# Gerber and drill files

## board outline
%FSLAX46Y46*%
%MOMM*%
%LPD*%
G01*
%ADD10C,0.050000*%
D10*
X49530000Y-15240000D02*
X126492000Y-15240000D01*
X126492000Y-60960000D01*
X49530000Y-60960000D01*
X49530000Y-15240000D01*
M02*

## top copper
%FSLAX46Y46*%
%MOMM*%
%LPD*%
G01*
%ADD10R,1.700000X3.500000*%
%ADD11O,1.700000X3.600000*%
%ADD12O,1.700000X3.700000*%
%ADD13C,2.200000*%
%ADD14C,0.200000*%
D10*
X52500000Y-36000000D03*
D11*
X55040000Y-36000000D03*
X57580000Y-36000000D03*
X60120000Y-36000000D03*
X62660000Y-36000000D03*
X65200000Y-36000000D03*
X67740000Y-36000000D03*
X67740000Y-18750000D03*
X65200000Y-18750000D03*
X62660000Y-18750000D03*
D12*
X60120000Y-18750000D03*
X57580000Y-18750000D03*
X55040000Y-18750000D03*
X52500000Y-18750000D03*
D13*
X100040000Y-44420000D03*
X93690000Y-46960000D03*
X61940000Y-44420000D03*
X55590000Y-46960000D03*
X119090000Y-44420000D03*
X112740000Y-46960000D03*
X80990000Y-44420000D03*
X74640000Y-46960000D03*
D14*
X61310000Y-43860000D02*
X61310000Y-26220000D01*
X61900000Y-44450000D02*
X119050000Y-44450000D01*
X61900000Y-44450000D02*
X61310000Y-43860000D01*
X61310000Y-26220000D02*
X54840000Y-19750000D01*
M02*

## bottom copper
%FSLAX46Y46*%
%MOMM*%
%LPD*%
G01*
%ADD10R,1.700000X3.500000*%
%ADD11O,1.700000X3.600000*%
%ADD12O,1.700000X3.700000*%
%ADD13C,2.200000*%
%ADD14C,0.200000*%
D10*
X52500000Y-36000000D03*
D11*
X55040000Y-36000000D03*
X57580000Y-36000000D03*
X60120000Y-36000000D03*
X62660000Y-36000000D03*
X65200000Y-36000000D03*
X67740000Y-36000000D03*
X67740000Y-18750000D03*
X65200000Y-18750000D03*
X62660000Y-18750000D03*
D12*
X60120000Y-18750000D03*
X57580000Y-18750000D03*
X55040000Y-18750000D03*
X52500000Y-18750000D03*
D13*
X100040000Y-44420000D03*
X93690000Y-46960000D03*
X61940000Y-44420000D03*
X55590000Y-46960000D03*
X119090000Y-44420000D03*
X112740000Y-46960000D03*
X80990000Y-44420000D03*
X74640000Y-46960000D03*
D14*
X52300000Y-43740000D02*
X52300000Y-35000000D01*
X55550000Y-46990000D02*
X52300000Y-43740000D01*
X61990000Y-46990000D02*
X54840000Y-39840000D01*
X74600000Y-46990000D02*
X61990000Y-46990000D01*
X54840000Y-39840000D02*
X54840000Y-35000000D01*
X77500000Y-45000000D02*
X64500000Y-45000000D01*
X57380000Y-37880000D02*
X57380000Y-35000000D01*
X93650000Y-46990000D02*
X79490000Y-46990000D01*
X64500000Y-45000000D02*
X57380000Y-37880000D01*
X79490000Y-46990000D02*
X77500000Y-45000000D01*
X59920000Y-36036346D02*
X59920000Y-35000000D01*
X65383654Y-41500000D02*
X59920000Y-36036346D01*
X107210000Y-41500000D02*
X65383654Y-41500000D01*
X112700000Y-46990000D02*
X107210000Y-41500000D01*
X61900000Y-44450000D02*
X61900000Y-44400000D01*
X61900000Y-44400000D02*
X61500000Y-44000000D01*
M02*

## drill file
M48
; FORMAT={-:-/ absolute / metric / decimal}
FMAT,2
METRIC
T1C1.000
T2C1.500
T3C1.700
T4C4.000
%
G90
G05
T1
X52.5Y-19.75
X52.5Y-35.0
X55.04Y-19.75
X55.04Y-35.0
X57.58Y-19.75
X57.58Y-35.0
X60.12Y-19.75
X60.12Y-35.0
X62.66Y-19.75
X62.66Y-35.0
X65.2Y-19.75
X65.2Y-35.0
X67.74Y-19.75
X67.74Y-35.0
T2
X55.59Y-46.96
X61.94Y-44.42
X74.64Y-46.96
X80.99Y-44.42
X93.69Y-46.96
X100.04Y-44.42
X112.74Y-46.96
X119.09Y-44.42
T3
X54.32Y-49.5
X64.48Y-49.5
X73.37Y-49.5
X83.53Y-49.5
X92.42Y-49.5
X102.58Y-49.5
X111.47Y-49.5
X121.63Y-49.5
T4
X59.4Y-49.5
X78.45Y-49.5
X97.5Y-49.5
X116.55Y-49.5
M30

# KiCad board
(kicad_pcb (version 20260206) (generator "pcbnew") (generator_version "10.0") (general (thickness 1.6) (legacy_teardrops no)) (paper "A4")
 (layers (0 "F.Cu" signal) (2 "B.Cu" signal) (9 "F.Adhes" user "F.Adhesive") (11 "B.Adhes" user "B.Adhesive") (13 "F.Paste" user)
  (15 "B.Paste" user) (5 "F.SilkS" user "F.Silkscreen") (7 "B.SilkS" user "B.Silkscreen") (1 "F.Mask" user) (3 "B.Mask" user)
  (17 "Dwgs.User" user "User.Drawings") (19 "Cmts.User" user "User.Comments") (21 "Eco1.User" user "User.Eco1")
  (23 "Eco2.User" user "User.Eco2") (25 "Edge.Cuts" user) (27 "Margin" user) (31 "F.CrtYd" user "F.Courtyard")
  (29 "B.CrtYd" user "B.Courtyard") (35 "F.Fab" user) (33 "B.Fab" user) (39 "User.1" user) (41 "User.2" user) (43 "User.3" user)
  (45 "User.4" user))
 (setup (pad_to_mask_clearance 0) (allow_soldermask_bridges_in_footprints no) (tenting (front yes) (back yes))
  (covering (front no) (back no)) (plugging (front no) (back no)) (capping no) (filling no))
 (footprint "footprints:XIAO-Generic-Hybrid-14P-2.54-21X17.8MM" (layer "F.Cu") (at 60.12 27.375 90)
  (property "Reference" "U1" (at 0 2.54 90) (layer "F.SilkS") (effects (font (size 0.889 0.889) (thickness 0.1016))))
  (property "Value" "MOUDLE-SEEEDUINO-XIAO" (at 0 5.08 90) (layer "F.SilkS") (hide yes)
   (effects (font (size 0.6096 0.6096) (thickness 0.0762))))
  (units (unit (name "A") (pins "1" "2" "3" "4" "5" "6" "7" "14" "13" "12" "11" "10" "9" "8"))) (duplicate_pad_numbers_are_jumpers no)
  (pad "1" thru_hole rect (at -7.625 -7.62 90) (size 3.5 1.7) (drill 1 (offset -1 0)) (layers "*.Cu" "*.Mask") (remove_unused_layers no)
   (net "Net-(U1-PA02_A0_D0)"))
  (pad "2" thru_hole oval (at -7.625 -5.08 90) (size 3.6 1.7) (drill 1 (offset -1 0)) (layers "*.Cu" "*.Mask") (remove_unused_layers no)
   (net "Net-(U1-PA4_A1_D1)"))
  (pad "3" thru_hole oval (at -7.625 -2.54 90) (size 3.6 1.7) (drill 1 (offset -1 0)) (layers "*.Cu" "*.Mask") (remove_unused_layers no)
   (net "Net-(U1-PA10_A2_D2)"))
  (pad "4" thru_hole oval (at -7.625 0 90) (size 3.6 1.7) (drill 1 (offset -1 0)) (layers "*.Cu" "*.Mask") (remove_unused_layers no)
   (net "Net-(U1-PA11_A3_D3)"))
  (pad "5" thru_hole oval (at -7.625 2.54 90) (size 3.6 1.7) (drill 1 (offset -1 0)) (layers "*.Cu" "*.Mask") (remove_unused_layers no)
   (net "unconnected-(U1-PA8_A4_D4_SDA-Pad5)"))
  (pad "6" thru_hole oval (at -7.625 5.08 270) (size 3.6 1.7) (drill 1 (offset 1 0)) (layers "*.Cu" "*.Mask") (remove_unused_layers no)
   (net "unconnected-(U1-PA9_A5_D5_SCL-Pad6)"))
  (pad "7" thru_hole oval (at -7.625 7.62 90) (size 3.6 1.7) (drill 1 (offset -1 0)) (layers "*.Cu" "*.Mask") (remove_unused_layers no)
   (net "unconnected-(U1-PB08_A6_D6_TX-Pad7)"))
  (pad "8" thru_hole oval (at 7.625 7.62 90) (size 3.6 1.7) (drill 1 (offset 1 0)) (layers "*.Cu" "*.Mask") (remove_unused_layers no)
   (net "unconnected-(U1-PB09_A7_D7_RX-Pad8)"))
  (pad "9" thru_hole oval (at 7.625 5.08 90) (size 3.6 1.7) (drill 1 (offset 1 0)) (layers "*.Cu" "*.Mask") (remove_unused_layers no)
   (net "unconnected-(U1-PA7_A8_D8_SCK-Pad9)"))
  (pad "10" thru_hole oval (at 7.625 2.54 90) (size 3.6 1.7) (drill 1 (offset 1 0)) (layers "*.Cu" "*.Mask") (remove_unused_layers no)
   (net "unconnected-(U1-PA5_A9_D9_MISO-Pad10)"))
  (pad "11" thru_hole oval (at 7.625 0 90) (size 3.7 1.7) (drill 1 (offset 1 0)) (layers "*.Cu" "*.Mask") (remove_unused_layers no)
   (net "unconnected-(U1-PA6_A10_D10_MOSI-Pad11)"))
  (pad "12" thru_hole oval (at 7.625 -2.54 90) (size 3.7 1.7) (drill 1 (offset 1 0)) (layers "*.Cu" "*.Mask") (remove_unused_layers no)
   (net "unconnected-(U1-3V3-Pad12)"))
  (pad "13" thru_hole oval (at 7.625 -5.08 90) (size 3.7 1.7) (drill 1 (offset 1 0)) (layers "*.Cu" "*.Mask") (remove_unused_layers no)
   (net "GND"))
  (pad "14" thru_hole oval (at 7.625 -7.62 90) (size 3.7 1.7) (drill 1 (offset 1 0)) (layers "*.Cu" "*.Mask") (remove_unused_layers no)
   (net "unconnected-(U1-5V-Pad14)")))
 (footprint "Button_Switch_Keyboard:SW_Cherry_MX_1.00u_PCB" (layer "F.Cu") (at 100.04 44.42)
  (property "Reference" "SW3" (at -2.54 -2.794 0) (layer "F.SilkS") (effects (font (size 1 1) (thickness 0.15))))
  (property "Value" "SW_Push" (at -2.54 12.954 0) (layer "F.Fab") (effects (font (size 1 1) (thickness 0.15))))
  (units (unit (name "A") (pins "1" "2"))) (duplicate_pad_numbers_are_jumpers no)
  (pad "" np_thru_hole circle (at -7.62 5.08) (size 1.7 1.7) (drill 1.7) (layers "*.Cu" "*.Mask"))
  (pad "" np_thru_hole circle (at -2.54 5.08) (size 4 4) (drill 4) (layers "*.Cu" "*.Mask"))
  (pad "" np_thru_hole circle (at 2.54 5.08) (size 1.7 1.7) (drill 1.7) (layers "*.Cu" "*.Mask"))
  (pad "1" thru_hole circle (at 0 0) (size 2.2 2.2) (drill 1.5) (layers "*.Cu" "*.Mask") (remove_unused_layers no) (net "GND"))
  (pad "2" thru_hole circle (at -6.35 2.54) (size 2.2 2.2) (drill 1.5) (layers "*.Cu" "*.Mask") (remove_unused_layers no)
   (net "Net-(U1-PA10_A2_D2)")))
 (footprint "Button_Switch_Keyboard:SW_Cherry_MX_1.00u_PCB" (layer "F.Cu") (at 61.94 44.42)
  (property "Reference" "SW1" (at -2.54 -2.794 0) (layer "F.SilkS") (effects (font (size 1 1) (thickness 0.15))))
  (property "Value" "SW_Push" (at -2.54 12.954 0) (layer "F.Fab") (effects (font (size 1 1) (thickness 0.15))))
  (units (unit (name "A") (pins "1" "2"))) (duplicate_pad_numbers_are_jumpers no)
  (pad "" np_thru_hole circle (at -7.62 5.08) (size 1.7 1.7) (drill 1.7) (layers "*.Cu" "*.Mask"))
  (pad "" np_thru_hole circle (at -2.54 5.08) (size 4 4) (drill 4) (layers "*.Cu" "*.Mask"))
  (pad "" np_thru_hole circle (at 2.54 5.08) (size 1.7 1.7) (drill 1.7) (layers "*.Cu" "*.Mask"))
  (pad "1" thru_hole circle (at 0 0) (size 2.2 2.2) (drill 1.5) (layers "*.Cu" "*.Mask") (remove_unused_layers no) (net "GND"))
  (pad "2" thru_hole circle (at -6.35 2.54) (size 2.2 2.2) (drill 1.5) (layers "*.Cu" "*.Mask") (remove_unused_layers no)
   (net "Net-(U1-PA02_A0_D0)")))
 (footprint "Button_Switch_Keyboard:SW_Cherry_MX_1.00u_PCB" (layer "F.Cu") (at 119.09 44.42)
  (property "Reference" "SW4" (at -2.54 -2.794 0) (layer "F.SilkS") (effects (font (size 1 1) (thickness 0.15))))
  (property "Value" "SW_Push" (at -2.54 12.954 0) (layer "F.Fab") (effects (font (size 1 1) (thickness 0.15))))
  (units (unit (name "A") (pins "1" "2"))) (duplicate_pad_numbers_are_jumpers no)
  (pad "" np_thru_hole circle (at -7.62 5.08) (size 1.7 1.7) (drill 1.7) (layers "*.Cu" "*.Mask"))
  (pad "" np_thru_hole circle (at -2.54 5.08) (size 4 4) (drill 4) (layers "*.Cu" "*.Mask"))
  (pad "" np_thru_hole circle (at 2.54 5.08) (size 1.7 1.7) (drill 1.7) (layers "*.Cu" "*.Mask"))
  (pad "1" thru_hole circle (at 0 0) (size 2.2 2.2) (drill 1.5) (layers "*.Cu" "*.Mask") (remove_unused_layers no) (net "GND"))
  (pad "2" thru_hole circle (at -6.35 2.54) (size 2.2 2.2) (drill 1.5) (layers "*.Cu" "*.Mask") (remove_unused_layers no)
   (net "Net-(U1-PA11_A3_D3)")))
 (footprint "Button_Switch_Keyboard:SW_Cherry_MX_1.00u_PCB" (layer "F.Cu") (at 80.99 44.42)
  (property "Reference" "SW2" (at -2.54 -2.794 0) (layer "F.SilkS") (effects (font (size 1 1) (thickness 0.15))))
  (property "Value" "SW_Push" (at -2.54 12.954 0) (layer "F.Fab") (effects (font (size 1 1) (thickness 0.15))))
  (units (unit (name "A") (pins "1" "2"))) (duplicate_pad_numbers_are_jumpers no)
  (pad "" np_thru_hole circle (at -7.62 5.08) (size 1.7 1.7) (drill 1.7) (layers "*.Cu" "*.Mask"))
  (pad "" np_thru_hole circle (at -2.54 5.08) (size 4 4) (drill 4) (layers "*.Cu" "*.Mask"))
  (pad "" np_thru_hole circle (at 2.54 5.08) (size 1.7 1.7) (drill 1.7) (layers "*.Cu" "*.Mask"))
  (pad "1" thru_hole circle (at 0 0) (size 2.2 2.2) (drill 1.5) (layers "*.Cu" "*.Mask") (remove_unused_layers no) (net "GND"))
  (pad "2" thru_hole circle (at -6.35 2.54) (size 2.2 2.2) (drill 1.5) (layers "*.Cu" "*.Mask") (remove_unused_layers no)
   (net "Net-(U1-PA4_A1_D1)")))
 (gr_rect (start 49.53 15.24) (end 126.492 60.96) (stroke (width 0.05) (type solid)) (fill no) (layer "Edge.Cuts"))
 (segment (start 52.3 43.74) (end 52.3 35) (width 0.2) (layer "B.Cu") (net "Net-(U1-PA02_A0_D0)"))
 (segment (start 55.55 46.99) (end 52.3 43.74) (width 0.2) (layer "B.Cu") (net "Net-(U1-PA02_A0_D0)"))
 (segment (start 61.99 46.99) (end 54.84 39.84) (width 0.2) (layer "B.Cu") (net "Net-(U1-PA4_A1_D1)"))
 (segment (start 74.6 46.99) (end 61.99 46.99) (width 0.2) (layer "B.Cu") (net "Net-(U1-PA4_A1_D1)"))
 (segment (start 54.84 39.84) (end 54.84 35) (width 0.2) (layer "B.Cu") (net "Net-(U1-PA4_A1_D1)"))
 (segment (start 77.5 45) (end 64.5 45) (width 0.2) (layer "B.Cu") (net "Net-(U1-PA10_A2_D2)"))
 (segment (start 57.38 37.88) (end 57.38 35) (width 0.2) (layer "B.Cu") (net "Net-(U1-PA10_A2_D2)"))
 (segment (start 93.65 46.99) (end 79.49 46.99) (width 0.2) (layer "B.Cu") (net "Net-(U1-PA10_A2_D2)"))
 (segment (start 64.5 45) (end 57.38 37.88) (width 0.2) (layer "B.Cu") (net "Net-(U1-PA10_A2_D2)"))
 (segment (start 79.49 46.99) (end 77.5 45) (width 0.2) (layer "B.Cu") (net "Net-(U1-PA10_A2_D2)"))
 (segment (start 59.92 36.036346) (end 59.92 35) (width 0.2) (layer "B.Cu") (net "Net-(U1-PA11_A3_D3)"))
 (segment (start 65.383654 41.5) (end 59.92 36.036346) (width 0.2) (layer "B.Cu") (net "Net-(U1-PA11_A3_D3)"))
 (segment (start 107.21 41.5) (end 65.383654 41.5) (width 0.2) (layer "B.Cu") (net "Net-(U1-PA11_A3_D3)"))
 (segment (start 112.7 46.99) (end 107.21 41.5) (width 0.2) (layer "B.Cu") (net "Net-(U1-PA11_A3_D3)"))
 (segment (start 61.31 43.86) (end 61.31 26.22) (width 0.2) (layer "F.Cu") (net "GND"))
 (segment (start 61.9 44.45) (end 119.05 44.45) (width 0.2) (layer "F.Cu") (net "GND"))
 (segment (start 61.9 44.45) (end 61.31 43.86) (width 0.2) (layer "F.Cu") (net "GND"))
 (segment (start 61.31 26.22) (end 54.84 19.75) (width 0.2) (layer "F.Cu") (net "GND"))
 (segment (start 61.9 44.45) (end 61.9 44.4) (width 0.2) (layer "B.Cu") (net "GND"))
 (segment (start 61.9 44.4) (end 61.5 44) (width 0.2) (layer "B.Cu") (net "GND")))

